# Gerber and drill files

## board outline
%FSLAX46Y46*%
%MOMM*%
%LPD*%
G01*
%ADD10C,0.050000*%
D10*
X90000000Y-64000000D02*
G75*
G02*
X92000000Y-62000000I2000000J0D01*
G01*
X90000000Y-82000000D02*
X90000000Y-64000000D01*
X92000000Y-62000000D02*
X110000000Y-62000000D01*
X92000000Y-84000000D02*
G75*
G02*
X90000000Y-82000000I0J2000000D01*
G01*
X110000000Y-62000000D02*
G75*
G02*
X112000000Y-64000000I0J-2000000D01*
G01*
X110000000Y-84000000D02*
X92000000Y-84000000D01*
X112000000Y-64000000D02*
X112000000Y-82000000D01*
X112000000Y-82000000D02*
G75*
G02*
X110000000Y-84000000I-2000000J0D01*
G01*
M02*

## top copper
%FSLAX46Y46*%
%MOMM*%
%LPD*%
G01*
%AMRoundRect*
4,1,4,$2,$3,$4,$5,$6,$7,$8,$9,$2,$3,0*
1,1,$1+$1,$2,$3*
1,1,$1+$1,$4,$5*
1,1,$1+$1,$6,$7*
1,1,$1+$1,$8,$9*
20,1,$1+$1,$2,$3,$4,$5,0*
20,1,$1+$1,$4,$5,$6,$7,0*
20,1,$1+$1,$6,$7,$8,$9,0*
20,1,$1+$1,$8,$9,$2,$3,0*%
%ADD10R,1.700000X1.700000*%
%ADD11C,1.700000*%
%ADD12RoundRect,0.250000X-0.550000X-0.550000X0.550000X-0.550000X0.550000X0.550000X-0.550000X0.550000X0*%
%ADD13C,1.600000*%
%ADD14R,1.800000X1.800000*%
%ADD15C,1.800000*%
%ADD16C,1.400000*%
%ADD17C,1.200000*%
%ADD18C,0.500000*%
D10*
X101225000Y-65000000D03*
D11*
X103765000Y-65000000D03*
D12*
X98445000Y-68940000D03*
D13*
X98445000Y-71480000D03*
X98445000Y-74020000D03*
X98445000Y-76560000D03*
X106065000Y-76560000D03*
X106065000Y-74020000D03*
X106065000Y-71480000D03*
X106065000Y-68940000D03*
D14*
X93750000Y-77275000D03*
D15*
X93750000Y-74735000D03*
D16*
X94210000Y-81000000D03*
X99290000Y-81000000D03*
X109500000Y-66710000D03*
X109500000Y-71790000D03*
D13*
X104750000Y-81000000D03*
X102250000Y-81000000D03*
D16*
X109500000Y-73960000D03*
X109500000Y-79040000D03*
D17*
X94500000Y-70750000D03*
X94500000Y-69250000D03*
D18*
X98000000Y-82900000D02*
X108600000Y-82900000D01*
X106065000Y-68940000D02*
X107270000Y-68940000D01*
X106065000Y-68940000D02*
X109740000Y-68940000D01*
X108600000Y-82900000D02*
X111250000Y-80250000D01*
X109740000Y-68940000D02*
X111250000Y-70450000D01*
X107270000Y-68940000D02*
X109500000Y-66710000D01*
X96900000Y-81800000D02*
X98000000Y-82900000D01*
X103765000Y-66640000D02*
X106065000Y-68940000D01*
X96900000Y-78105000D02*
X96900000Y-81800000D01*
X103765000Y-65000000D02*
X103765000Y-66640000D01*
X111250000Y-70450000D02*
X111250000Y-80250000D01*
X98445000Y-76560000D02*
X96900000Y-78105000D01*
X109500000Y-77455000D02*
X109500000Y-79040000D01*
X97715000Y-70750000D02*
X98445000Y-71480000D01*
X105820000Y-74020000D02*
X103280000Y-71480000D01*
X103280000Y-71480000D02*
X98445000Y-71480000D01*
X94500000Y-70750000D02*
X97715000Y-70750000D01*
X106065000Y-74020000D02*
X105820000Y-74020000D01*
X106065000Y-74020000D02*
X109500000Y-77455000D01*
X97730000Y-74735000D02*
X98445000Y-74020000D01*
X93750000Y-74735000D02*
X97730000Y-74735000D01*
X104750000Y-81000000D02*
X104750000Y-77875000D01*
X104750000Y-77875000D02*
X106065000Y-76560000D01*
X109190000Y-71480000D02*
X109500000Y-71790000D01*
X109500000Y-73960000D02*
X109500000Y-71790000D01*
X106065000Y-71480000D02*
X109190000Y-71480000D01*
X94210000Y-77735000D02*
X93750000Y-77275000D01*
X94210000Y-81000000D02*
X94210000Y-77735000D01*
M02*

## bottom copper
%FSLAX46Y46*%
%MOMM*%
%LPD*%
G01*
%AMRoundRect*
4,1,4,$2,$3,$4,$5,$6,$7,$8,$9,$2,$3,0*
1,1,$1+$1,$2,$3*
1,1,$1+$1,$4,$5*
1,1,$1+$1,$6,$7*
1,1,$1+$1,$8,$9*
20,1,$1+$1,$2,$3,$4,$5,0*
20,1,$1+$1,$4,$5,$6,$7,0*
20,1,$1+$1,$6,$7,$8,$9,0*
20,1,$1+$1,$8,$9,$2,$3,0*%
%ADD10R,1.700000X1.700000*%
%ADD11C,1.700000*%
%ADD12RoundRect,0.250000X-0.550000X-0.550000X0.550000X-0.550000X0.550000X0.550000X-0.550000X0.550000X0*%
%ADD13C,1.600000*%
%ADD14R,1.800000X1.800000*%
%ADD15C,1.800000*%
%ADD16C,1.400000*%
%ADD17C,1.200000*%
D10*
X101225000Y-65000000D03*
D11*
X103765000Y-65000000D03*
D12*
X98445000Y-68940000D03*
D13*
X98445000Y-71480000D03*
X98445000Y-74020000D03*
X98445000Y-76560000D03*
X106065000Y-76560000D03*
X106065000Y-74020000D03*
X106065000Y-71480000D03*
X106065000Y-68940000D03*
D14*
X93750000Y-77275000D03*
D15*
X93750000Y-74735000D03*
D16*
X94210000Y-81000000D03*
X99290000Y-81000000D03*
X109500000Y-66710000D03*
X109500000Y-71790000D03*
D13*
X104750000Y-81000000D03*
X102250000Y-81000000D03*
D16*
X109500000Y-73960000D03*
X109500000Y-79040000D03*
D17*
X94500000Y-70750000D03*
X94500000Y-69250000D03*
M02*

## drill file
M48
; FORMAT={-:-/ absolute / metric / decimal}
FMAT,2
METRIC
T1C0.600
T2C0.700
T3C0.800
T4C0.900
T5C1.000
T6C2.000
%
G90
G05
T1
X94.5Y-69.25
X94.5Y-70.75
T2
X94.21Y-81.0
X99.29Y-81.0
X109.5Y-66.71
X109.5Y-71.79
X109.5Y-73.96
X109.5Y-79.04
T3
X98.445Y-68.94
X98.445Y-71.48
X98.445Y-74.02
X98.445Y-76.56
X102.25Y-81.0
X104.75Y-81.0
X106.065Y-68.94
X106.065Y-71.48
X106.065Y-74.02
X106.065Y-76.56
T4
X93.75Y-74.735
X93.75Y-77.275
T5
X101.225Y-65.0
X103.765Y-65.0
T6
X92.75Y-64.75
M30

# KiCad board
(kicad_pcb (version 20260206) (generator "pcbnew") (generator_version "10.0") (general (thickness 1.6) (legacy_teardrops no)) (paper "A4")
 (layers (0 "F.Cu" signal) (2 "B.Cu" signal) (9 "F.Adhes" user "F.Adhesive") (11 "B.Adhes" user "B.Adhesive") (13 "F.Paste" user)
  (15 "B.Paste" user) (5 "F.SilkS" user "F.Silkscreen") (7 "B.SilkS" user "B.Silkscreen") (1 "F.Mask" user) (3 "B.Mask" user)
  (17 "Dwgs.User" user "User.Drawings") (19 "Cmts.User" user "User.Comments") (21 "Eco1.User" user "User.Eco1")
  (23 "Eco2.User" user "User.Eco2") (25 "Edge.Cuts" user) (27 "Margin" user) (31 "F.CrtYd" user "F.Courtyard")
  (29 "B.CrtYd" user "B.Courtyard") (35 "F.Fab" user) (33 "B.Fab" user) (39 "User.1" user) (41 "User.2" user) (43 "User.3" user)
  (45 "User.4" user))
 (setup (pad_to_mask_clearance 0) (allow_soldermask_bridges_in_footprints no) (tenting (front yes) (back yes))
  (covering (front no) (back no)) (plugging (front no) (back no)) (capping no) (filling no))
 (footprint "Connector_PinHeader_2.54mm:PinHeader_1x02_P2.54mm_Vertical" (layer "F.Cu") (at 101.225 65 90)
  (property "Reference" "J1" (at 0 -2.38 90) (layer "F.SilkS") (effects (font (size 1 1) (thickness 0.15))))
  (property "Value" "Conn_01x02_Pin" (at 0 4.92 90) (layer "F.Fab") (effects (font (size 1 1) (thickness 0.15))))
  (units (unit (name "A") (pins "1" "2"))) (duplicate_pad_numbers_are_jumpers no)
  (pad "1" thru_hole rect (at 0 0 90) (size 1.7 1.7) (drill 1) (layers "*.Cu" "*.Mask") (remove_unused_layers no) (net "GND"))
  (pad "2" thru_hole circle (at 0 2.54 90) (size 1.7 1.7) (drill 1) (layers "*.Cu" "*.Mask") (remove_unused_layers no) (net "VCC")))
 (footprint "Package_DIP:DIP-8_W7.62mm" (layer "F.Cu") (at 98.445 68.94)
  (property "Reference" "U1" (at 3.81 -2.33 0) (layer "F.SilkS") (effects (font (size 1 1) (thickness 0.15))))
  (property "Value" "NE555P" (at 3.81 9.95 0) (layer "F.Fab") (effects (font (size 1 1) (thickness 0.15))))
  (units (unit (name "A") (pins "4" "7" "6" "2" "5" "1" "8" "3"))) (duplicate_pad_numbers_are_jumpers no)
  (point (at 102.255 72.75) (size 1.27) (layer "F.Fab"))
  (pad "1" thru_hole roundrect (at 0 0) (size 1.6 1.6) (drill 0.8) (layers "*.Cu" "*.Mask") (remove_unused_layers no)
   (roundrect_rratio 0.15625) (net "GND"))
  (pad "2" thru_hole circle (at 0 2.54) (size 1.6 1.6) (drill 0.8) (layers "*.Cu" "*.Mask") (remove_unused_layers no) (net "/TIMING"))
  (pad "3" thru_hole circle (at 0 5.08) (size 1.6 1.6) (drill 0.8) (layers "*.Cu" "*.Mask") (remove_unused_layers no) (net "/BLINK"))
  (pad "4" thru_hole circle (at 0 7.62) (size 1.6 1.6) (drill 0.8) (layers "*.Cu" "*.Mask") (remove_unused_layers no) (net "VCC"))
  (pad "5" thru_hole circle (at 7.62 7.62) (size 1.6 1.6) (drill 0.8) (layers "*.Cu" "*.Mask") (remove_unused_layers no)
   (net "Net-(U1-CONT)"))
  (pad "6" thru_hole circle (at 7.62 5.08) (size 1.6 1.6) (drill 0.8) (layers "*.Cu" "*.Mask") (remove_unused_layers no) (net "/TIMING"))
  (pad "7" thru_hole circle (at 7.62 2.54) (size 1.6 1.6) (drill 0.8) (layers "*.Cu" "*.Mask") (remove_unused_layers no) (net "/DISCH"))
  (pad "8" thru_hole circle (at 7.62 0) (size 1.6 1.6) (drill 0.8) (layers "*.Cu" "*.Mask") (remove_unused_layers no) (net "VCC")))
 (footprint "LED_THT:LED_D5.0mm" (layer "F.Cu") (at 93.75 77.275 90)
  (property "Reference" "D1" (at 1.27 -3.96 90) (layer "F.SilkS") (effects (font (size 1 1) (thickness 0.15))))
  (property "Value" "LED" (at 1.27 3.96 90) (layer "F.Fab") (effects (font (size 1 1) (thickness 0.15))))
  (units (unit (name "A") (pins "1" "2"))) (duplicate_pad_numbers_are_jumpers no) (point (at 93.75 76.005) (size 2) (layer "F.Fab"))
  (pad "1" thru_hole rect (at 0 0 90) (size 1.8 1.8) (drill 0.9) (layers "*.Cu" "*.Mask") (remove_unused_layers no) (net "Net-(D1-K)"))
  (pad "2" thru_hole circle (at 2.54 0 90) (size 1.8 1.8) (drill 0.9) (layers "*.Cu" "*.Mask") (remove_unused_layers no) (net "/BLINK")))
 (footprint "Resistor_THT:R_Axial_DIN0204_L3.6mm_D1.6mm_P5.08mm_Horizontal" (layer "F.Cu") (at 94.21 81)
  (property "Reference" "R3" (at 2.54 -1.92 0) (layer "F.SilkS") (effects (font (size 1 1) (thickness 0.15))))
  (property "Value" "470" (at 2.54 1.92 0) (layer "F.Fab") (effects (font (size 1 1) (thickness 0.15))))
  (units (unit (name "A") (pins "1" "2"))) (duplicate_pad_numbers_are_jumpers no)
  (pad "1" thru_hole circle (at 0 0) (size 1.4 1.4) (drill 0.7) (layers "*.Cu" "*.Mask") (remove_unused_layers no) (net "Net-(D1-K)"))
  (pad "2" thru_hole circle (at 5.08 0) (size 1.4 1.4) (drill 0.7) (layers "*.Cu" "*.Mask") (remove_unused_layers no) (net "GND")))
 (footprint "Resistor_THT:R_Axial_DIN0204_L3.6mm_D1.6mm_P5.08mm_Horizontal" (layer "F.Cu") (at 109.5 66.71 -90)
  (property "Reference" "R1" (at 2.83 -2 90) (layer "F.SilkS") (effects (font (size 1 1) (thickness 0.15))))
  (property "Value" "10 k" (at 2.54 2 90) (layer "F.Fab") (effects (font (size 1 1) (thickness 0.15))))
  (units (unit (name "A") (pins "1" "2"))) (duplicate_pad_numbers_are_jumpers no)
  (pad "1" thru_hole circle (at 0 0 270) (size 1.4 1.4) (drill 0.7) (layers "*.Cu" "*.Mask") (remove_unused_layers no) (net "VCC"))
  (pad "2" thru_hole circle (at 5.08 0 270) (size 1.4 1.4) (drill 0.7) (layers "*.Cu" "*.Mask") (remove_unused_layers no) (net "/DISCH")))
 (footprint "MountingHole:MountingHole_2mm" (layer "F.Cu") (at 92.75 64.75)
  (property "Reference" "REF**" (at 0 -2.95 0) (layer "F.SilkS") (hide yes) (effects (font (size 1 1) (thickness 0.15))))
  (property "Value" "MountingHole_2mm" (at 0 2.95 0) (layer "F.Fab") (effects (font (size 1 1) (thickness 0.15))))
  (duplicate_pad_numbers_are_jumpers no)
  (pad "" np_thru_hole circle (at 0 0) (size 2 2) (drill 2) (layers "*.Cu" "*.Mask")))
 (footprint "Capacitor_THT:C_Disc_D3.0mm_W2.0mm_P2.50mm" (layer "F.Cu") (at 104.75 81 180)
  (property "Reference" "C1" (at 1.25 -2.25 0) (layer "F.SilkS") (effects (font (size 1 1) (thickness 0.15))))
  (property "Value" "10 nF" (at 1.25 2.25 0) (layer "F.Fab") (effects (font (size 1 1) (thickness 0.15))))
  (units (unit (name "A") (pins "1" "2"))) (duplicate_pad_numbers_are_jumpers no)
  (pad "1" thru_hole circle (at 0 0 180) (size 1.6 1.6) (drill 0.8) (layers "*.Cu" "*.Mask") (remove_unused_layers no) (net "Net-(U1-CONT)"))
  (pad "2" thru_hole circle (at 2.5 0 180) (size 1.6 1.6) (drill 0.8) (layers "*.Cu" "*.Mask") (remove_unused_layers no) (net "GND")))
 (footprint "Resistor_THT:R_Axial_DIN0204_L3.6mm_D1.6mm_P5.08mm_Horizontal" (layer "F.Cu") (at 109.5 73.96 -90)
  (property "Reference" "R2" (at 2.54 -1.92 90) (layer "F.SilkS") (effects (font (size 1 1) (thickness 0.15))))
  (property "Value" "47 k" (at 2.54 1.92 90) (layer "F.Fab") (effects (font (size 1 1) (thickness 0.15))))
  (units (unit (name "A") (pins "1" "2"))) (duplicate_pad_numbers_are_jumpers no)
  (pad "1" thru_hole circle (at 0 0 270) (size 1.4 1.4) (drill 0.7) (layers "*.Cu" "*.Mask") (remove_unused_layers no) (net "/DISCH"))
  (pad "2" thru_hole circle (at 5.08 0 270) (size 1.4 1.4) (drill 0.7) (layers "*.Cu" "*.Mask") (remove_unused_layers no) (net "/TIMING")))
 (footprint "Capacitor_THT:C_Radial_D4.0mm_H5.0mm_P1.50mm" (layer "F.Cu") (at 94.5 70.75 90)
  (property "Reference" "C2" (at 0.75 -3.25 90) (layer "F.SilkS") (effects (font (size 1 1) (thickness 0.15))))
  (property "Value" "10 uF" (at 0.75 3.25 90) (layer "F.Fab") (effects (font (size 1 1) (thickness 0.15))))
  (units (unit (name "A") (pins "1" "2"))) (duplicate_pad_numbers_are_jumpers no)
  (pad "1" thru_hole circle (at 0 0 90) (size 1.2 1.2) (drill 0.6) (layers "*.Cu" "*.Mask") (remove_unused_layers no) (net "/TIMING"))
  (pad "2" thru_hole circle (at 1.5 0 90) (size 1.2 1.2) (drill 0.6) (layers "*.Cu" "*.Mask") (remove_unused_layers no) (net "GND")))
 (gr_arc (start 90 64) (mid 90.585786 62.585786) (end 92 62) (stroke (width 0.05) (type default)) (layer "Edge.Cuts"))
 (gr_line (start 90 82) (end 90 64) (stroke (width 0.05) (type default)) (layer "Edge.Cuts"))
 (gr_line (start 92 62) (end 110 62) (stroke (width 0.05) (type default)) (layer "Edge.Cuts"))
 (gr_arc (start 92 84) (mid 90.585786 83.414214) (end 90 82) (stroke (width 0.05) (type default)) (layer "Edge.Cuts"))
 (gr_arc (start 110 62) (mid 111.414214 62.585786) (end 112 64) (stroke (width 0.05) (type default)) (layer "Edge.Cuts"))
 (gr_line (start 110 84) (end 92 84) (stroke (width 0.05) (type default)) (layer "Edge.Cuts"))
 (gr_line (start 112 64) (end 112 82) (stroke (width 0.05) (type default)) (layer "Edge.Cuts"))
 (gr_arc (start 112 82) (mid 111.414214 83.414214) (end 110 84) (stroke (width 0.05) (type default)) (layer "Edge.Cuts"))
 (segment (start 98 82.9) (end 108.6 82.9) (width 0.5) (layer "F.Cu") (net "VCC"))
 (segment (start 106.065 68.94) (end 107.27 68.94) (width 0.5) (layer "F.Cu") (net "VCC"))
 (segment (start 106.065 68.94) (end 109.74 68.94) (width 0.5) (layer "F.Cu") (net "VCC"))
 (segment (start 108.6 82.9) (end 111.25 80.25) (width 0.5) (layer "F.Cu") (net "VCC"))
 (segment (start 109.74 68.94) (end 111.25 70.45) (width 0.5) (layer "F.Cu") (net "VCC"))
 (segment (start 107.27 68.94) (end 109.5 66.71) (width 0.5) (layer "F.Cu") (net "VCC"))
 (segment (start 96.9 81.8) (end 98 82.9) (width 0.5) (layer "F.Cu") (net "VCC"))
 (segment (start 103.765 66.64) (end 106.065 68.94) (width 0.5) (layer "F.Cu") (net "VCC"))
 (segment (start 96.9 78.105) (end 96.9 81.8) (width 0.5) (layer "F.Cu") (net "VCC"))
 (segment (start 103.765 65) (end 103.765 66.64) (width 0.5) (layer "F.Cu") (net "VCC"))
 (segment (start 111.25 70.45) (end 111.25 80.25) (width 0.5) (layer "F.Cu") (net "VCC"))
 (segment (start 98.445 76.56) (end 96.9 78.105) (width 0.5) (layer "F.Cu") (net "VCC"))
 (segment (start 109.5 77.455) (end 109.5 79.04) (width 0.5) (layer "F.Cu") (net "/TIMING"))
 (segment (start 97.715 70.75) (end 98.445 71.48) (width 0.5) (layer "F.Cu") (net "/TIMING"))
 (segment (start 105.82 74.02) (end 103.28 71.48) (width 0.5) (layer "F.Cu") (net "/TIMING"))
 (segment (start 103.28 71.48) (end 98.445 71.48) (width 0.5) (layer "F.Cu") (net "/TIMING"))
 (segment (start 94.5 70.75) (end 97.715 70.75) (width 0.5) (layer "F.Cu") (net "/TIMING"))
 (segment (start 106.065 74.02) (end 105.82 74.02) (width 0.5) (layer "F.Cu") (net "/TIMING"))
 (segment (start 106.065 74.02) (end 109.5 77.455) (width 0.5) (layer "F.Cu") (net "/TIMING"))
 (segment (start 97.73 74.735) (end 98.445 74.02) (width 0.5) (layer "F.Cu") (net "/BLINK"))
 (segment (start 93.75 74.735) (end 97.73 74.735) (width 0.5) (layer "F.Cu") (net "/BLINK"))
 (segment (start 104.75 81) (end 104.75 77.875) (width 0.5) (layer "F.Cu") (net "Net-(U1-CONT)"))
 (segment (start 104.75 77.875) (end 106.065 76.56) (width 0.5) (layer "F.Cu") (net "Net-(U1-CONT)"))
 (segment (start 109.19 71.48) (end 109.5 71.79) (width 0.5) (layer "F.Cu") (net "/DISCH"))
 (segment (start 109.5 73.96) (end 109.5 71.79) (width 0.5) (layer "F.Cu") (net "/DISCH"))
 (segment (start 106.065 71.48) (end 109.19 71.48) (width 0.5) (layer "F.Cu") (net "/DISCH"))
 (segment (start 94.21 77.735) (end 93.75 77.275) (width 0.5) (layer "F.Cu") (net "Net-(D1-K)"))
 (segment (start 94.21 81) (end 94.21 77.735) (width 0.5) (layer "F.Cu") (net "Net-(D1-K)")))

